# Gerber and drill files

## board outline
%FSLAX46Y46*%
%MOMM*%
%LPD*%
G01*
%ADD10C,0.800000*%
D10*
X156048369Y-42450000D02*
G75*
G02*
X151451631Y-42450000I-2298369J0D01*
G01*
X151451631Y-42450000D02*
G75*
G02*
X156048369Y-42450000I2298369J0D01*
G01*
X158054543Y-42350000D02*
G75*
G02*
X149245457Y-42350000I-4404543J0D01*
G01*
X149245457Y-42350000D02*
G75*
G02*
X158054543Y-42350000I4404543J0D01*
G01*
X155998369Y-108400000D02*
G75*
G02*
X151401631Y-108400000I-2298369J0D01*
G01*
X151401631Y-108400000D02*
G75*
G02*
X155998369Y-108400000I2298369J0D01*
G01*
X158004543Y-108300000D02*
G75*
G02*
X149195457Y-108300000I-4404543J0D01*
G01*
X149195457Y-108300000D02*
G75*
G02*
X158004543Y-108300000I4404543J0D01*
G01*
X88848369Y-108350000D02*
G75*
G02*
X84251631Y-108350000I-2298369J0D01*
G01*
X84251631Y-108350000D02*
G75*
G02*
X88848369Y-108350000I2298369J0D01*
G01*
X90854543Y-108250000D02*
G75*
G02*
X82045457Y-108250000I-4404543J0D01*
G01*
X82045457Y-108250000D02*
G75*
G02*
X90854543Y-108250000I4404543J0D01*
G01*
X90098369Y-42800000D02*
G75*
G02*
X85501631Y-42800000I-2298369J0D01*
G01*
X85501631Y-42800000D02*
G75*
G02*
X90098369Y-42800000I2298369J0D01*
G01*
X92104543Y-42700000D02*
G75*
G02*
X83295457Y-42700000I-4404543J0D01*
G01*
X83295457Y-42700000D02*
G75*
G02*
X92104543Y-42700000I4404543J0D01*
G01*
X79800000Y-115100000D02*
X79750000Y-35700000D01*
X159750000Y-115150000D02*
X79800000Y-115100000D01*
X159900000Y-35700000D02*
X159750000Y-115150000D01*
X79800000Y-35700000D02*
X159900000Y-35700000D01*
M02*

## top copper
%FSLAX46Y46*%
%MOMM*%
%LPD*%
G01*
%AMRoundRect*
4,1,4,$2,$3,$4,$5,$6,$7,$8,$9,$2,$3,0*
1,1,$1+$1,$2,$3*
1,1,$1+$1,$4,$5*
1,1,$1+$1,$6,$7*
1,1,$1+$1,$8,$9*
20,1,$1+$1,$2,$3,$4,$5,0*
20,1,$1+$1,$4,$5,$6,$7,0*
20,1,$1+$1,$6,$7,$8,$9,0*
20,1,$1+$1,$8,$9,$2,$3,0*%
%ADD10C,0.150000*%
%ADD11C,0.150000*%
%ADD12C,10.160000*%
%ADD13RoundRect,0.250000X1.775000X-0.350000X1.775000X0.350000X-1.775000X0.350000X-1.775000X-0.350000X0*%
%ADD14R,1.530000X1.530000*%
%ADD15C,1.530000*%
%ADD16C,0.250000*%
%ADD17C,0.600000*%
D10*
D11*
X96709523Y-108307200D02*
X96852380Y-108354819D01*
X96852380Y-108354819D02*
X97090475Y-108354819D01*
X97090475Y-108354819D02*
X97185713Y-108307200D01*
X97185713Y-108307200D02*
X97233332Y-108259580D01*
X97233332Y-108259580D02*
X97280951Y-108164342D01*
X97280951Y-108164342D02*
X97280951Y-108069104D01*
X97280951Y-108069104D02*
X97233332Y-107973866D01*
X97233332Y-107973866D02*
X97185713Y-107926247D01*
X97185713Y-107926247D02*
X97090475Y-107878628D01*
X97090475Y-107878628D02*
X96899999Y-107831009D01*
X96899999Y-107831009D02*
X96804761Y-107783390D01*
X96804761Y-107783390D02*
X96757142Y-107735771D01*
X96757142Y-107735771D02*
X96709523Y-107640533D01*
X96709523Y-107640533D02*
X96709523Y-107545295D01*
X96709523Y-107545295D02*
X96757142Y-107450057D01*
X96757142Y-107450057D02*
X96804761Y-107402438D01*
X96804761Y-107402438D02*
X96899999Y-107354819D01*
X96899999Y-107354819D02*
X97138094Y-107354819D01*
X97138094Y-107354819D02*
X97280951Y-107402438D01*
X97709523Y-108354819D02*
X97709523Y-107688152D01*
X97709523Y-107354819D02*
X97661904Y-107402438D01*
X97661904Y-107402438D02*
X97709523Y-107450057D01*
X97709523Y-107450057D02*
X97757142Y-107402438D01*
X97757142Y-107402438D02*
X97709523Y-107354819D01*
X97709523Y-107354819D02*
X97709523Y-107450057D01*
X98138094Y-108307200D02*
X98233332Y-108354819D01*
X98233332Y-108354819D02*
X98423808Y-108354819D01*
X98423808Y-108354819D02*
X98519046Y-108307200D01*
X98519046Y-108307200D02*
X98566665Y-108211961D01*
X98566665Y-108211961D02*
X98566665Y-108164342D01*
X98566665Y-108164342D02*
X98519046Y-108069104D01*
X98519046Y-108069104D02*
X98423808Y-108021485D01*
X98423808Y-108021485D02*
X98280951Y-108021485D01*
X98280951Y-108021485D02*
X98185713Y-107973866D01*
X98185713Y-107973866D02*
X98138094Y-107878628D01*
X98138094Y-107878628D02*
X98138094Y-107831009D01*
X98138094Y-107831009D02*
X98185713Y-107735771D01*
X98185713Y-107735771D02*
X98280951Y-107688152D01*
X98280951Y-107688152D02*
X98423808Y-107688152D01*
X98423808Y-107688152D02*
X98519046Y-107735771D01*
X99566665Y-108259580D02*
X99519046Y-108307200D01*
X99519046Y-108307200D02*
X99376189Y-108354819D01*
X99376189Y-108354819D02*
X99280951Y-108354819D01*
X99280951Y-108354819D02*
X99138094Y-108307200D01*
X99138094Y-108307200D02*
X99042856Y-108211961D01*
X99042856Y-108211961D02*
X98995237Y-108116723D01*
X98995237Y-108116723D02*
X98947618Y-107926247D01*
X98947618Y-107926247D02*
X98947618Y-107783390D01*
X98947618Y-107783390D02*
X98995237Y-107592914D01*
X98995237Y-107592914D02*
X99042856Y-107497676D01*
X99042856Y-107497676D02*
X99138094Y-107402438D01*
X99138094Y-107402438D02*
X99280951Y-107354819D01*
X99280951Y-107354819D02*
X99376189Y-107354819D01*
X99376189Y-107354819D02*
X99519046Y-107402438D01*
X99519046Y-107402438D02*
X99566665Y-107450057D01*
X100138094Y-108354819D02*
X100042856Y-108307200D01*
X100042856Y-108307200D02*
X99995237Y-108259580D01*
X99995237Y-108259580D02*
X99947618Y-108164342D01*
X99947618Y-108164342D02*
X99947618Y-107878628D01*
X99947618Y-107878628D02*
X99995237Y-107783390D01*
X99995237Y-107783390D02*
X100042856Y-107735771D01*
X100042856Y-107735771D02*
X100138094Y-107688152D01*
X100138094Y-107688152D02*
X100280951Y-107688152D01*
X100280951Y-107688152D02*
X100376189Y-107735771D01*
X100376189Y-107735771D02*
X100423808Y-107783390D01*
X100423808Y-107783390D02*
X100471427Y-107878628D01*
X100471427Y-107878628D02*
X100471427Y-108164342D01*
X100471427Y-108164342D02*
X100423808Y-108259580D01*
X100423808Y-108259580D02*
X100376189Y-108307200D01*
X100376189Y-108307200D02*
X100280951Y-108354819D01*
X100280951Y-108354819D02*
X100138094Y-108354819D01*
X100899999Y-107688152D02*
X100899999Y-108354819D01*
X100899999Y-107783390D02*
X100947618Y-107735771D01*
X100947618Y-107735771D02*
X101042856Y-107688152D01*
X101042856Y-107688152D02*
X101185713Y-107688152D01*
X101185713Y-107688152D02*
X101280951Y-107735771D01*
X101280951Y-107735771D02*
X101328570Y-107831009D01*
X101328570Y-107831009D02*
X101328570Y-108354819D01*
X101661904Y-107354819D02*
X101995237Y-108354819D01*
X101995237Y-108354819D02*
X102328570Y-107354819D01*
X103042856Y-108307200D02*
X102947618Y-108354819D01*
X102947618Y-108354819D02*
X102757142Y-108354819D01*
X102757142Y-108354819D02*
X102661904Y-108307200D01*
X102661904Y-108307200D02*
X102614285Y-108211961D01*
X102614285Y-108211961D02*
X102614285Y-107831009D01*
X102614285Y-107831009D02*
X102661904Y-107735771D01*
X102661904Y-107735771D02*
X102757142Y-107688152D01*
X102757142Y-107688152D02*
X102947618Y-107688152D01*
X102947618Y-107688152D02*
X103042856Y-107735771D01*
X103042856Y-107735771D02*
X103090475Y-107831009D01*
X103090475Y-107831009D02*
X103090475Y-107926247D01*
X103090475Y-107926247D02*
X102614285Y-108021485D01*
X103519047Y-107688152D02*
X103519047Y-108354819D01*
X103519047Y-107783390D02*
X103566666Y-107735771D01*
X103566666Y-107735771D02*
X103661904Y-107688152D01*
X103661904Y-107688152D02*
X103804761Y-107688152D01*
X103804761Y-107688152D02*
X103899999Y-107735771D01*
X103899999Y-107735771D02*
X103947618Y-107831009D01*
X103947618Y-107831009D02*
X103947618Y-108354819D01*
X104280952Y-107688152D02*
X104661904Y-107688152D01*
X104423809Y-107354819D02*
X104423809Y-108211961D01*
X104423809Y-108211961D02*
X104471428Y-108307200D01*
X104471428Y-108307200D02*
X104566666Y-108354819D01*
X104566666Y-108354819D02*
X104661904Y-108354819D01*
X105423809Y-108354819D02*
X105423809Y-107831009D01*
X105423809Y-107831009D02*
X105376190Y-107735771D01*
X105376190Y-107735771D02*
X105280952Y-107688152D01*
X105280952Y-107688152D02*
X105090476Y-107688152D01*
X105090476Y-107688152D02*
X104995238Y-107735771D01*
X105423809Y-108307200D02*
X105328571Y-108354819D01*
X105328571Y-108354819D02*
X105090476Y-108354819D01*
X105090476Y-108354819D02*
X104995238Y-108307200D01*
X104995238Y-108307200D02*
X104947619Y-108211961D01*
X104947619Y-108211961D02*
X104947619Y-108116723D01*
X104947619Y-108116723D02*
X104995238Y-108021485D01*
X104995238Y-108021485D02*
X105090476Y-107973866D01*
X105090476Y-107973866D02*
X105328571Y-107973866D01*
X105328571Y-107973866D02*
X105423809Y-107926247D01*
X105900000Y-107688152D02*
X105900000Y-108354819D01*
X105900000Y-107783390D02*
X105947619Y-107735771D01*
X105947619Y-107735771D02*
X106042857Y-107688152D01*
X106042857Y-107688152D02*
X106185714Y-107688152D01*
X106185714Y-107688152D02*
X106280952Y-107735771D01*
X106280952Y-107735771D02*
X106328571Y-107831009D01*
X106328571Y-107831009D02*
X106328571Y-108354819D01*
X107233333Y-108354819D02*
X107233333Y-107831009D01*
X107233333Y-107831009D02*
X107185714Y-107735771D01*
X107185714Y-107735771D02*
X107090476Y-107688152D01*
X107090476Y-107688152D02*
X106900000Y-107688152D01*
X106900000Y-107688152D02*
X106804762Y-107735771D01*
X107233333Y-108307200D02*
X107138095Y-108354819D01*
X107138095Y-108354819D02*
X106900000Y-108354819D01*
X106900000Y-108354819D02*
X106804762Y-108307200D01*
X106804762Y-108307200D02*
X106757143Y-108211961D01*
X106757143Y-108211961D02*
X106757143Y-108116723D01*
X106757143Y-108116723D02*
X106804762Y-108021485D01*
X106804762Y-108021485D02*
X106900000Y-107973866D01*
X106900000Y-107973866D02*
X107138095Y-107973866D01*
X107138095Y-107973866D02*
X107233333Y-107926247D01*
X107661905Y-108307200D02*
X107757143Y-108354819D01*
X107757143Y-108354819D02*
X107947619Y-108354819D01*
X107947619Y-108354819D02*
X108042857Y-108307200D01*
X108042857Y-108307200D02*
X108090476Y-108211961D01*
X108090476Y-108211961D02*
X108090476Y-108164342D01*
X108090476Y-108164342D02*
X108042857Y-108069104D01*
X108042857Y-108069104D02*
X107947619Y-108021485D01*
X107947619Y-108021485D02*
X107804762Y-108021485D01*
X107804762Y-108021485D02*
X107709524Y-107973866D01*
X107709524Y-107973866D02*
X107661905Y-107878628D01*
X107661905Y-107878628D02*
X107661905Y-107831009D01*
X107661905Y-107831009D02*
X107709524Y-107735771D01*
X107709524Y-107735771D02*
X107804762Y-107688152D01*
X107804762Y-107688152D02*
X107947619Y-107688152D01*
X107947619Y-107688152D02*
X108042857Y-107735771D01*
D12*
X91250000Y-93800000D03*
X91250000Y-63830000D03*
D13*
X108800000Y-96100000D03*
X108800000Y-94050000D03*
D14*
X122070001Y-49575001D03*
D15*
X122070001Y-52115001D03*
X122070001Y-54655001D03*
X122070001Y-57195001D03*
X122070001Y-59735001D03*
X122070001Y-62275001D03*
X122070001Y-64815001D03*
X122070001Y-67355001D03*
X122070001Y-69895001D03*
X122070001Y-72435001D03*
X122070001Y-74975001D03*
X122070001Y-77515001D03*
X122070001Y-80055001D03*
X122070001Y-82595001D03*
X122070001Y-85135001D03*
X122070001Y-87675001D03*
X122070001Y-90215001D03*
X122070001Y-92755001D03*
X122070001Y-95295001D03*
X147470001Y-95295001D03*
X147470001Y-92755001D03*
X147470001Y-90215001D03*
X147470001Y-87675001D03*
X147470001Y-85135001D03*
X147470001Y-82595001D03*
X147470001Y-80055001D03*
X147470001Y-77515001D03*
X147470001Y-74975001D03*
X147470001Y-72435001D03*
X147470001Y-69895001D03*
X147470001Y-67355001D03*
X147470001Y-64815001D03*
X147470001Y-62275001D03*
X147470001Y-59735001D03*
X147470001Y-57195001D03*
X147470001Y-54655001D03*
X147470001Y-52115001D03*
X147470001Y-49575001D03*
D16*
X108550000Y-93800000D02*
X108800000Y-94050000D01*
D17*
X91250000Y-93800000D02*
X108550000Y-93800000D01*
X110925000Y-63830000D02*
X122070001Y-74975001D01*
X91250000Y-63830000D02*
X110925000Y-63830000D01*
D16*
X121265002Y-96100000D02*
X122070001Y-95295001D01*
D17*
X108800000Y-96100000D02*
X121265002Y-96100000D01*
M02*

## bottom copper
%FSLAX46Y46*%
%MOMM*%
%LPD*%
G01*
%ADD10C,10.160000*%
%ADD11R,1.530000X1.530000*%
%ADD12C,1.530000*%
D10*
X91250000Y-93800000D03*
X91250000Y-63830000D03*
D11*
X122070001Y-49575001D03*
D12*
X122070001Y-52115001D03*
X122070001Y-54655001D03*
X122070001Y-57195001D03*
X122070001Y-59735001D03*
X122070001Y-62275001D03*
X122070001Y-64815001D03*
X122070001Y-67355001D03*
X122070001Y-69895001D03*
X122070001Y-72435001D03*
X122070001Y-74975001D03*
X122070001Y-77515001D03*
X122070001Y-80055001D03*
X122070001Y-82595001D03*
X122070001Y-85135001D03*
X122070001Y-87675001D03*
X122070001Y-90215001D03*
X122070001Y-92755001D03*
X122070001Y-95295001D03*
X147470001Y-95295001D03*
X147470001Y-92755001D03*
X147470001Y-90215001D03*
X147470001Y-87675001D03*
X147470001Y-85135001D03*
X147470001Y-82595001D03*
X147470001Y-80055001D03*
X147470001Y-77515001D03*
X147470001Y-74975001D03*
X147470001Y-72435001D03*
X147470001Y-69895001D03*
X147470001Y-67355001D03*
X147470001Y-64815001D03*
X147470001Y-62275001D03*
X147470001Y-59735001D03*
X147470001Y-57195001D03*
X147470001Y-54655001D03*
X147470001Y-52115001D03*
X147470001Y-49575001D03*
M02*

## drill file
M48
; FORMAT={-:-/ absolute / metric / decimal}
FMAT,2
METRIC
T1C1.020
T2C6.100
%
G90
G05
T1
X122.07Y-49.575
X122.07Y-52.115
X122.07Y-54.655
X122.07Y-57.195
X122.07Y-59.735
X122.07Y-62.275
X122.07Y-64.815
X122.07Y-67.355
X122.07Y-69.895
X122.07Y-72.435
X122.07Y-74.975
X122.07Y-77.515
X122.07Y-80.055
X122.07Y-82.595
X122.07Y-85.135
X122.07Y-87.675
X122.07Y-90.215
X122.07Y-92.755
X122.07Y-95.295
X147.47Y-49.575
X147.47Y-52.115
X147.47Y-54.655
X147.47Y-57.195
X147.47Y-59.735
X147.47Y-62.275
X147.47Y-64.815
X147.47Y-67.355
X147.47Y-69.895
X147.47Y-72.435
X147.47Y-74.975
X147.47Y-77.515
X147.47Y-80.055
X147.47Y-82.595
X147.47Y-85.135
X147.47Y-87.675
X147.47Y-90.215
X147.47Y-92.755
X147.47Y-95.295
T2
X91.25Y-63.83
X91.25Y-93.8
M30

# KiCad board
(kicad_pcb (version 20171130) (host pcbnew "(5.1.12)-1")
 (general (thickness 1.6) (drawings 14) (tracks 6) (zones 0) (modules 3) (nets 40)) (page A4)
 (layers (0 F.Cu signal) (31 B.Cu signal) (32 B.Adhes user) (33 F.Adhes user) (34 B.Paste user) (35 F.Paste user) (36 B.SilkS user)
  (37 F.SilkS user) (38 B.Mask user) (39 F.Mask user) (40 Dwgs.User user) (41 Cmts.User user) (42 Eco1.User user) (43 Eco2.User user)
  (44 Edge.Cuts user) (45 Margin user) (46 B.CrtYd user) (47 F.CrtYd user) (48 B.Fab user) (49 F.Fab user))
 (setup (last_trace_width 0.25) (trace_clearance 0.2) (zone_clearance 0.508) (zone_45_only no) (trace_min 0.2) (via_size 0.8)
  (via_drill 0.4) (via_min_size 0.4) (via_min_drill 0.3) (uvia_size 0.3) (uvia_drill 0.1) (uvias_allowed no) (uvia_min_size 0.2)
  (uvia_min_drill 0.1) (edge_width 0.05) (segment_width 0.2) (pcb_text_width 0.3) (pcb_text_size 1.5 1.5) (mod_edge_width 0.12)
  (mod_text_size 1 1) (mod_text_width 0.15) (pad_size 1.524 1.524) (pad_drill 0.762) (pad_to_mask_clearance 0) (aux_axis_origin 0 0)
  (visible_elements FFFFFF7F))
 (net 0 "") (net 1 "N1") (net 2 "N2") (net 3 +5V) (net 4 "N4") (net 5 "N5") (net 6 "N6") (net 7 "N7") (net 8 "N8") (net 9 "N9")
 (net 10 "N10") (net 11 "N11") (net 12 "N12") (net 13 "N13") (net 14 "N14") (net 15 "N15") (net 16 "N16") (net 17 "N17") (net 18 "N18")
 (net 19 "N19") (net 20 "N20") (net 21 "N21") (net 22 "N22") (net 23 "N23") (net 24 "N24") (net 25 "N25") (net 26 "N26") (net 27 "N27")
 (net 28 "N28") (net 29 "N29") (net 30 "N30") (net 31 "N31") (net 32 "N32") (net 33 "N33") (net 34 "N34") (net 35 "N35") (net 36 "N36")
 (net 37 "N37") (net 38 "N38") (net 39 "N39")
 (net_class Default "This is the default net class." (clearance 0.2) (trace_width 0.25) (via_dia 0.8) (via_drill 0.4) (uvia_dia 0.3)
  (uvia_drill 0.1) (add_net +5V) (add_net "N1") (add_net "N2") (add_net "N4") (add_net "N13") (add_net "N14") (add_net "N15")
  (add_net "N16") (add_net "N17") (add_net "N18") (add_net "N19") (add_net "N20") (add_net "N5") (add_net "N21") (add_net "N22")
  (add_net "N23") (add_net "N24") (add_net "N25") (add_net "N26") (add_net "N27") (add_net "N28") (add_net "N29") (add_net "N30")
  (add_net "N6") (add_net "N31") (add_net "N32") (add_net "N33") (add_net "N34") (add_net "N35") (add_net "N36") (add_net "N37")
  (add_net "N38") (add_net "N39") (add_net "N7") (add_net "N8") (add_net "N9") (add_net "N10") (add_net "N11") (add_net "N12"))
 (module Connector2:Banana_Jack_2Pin (layer F.Cu) (at 91.25 93.8 90)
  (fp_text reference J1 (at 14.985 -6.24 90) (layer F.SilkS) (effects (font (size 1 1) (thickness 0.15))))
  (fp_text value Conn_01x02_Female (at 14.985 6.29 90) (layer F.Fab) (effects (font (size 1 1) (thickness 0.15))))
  (pad 1 thru_hole circle (at 0 0 90) (size 10.16 10.16) (drill 6.1) (layers *.Cu *.Mask) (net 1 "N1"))
  (pad 2 thru_hole circle (at 29.97 0 90) (size 10.16 10.16) (drill 6.1) (layers *.Cu *.Mask) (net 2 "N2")))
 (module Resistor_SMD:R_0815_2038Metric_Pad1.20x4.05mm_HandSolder (layer F.Cu) (at 108.8 95.075 90)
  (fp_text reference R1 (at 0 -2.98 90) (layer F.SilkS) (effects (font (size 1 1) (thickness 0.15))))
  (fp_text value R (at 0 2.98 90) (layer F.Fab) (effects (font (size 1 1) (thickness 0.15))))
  (pad 1 smd roundrect (at -1.025 0 90) (size 1.2 4.05) (layers F.Cu F.Paste F.Mask) (roundrect_rratio 0.208333) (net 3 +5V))
  (pad 2 smd roundrect (at 1.025 0 90) (size 1.2 4.05) (layers F.Cu F.Paste F.Mask) (roundrect_rratio 0.208333) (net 1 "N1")))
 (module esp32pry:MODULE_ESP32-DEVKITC (layer F.Cu) (at 134.770001 72.425001)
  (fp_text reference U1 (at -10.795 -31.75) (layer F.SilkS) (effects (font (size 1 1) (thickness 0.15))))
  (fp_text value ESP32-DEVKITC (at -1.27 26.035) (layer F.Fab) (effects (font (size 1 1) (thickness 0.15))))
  (pad 1 thru_hole rect (at -12.7 -22.85) (size 1.53 1.53) (drill 1.02) (layers *.Cu *.Mask) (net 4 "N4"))
  (pad 2 thru_hole circle (at -12.7 -20.31) (size 1.53 1.53) (drill 1.02) (layers *.Cu *.Mask) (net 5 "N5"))
  (pad 3 thru_hole circle (at -12.7 -17.77) (size 1.53 1.53) (drill 1.02) (layers *.Cu *.Mask) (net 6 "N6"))
  (pad 4 thru_hole circle (at -12.7 -15.23) (size 1.53 1.53) (drill 1.02) (layers *.Cu *.Mask) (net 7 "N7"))
  (pad 5 thru_hole circle (at -12.7 -12.69) (size 1.53 1.53) (drill 1.02) (layers *.Cu *.Mask) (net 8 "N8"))
  (pad 6 thru_hole circle (at -12.7 -10.15) (size 1.53 1.53) (drill 1.02) (layers *.Cu *.Mask) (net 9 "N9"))
  (pad 7 thru_hole circle (at -12.7 -7.61) (size 1.53 1.53) (drill 1.02) (layers *.Cu *.Mask) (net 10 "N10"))
  (pad 8 thru_hole circle (at -12.7 -5.07) (size 1.53 1.53) (drill 1.02) (layers *.Cu *.Mask) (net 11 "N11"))
  (pad 9 thru_hole circle (at -12.7 -2.53) (size 1.53 1.53) (drill 1.02) (layers *.Cu *.Mask) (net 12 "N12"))
  (pad 10 thru_hole circle (at -12.7 0.01) (size 1.53 1.53) (drill 1.02) (layers *.Cu *.Mask) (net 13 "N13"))
  (pad 11 thru_hole circle (at -12.7 2.55) (size 1.53 1.53) (drill 1.02) (layers *.Cu *.Mask) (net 2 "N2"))
  (pad 12 thru_hole circle (at -12.7 5.09) (size 1.53 1.53) (drill 1.02) (layers *.Cu *.Mask) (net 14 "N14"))
  (pad 13 thru_hole circle (at -12.7 7.63) (size 1.53 1.53) (drill 1.02) (layers *.Cu *.Mask) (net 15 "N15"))
  (pad 14 thru_hole circle (at -12.7 10.17) (size 1.53 1.53) (drill 1.02) (layers *.Cu *.Mask) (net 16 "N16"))
  (pad 15 thru_hole circle (at -12.7 12.71) (size 1.53 1.53) (drill 1.02) (layers *.Cu *.Mask) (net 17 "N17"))
  (pad 16 thru_hole circle (at -12.7 15.25) (size 1.53 1.53) (drill 1.02) (layers *.Cu *.Mask) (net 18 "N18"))
  (pad 17 thru_hole circle (at -12.7 17.79) (size 1.53 1.53) (drill 1.02) (layers *.Cu *.Mask) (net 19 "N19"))
  (pad 18 thru_hole circle (at -12.7 20.33) (size 1.53 1.53) (drill 1.02) (layers *.Cu *.Mask) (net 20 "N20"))
  (pad 19 thru_hole circle (at -12.7 22.87) (size 1.53 1.53) (drill 1.02) (layers *.Cu *.Mask) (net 3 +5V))
  (pad 20 thru_hole circle (at 12.7 22.87) (size 1.53 1.53) (drill 1.02) (layers *.Cu *.Mask) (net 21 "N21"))
  (pad 21 thru_hole circle (at 12.7 20.33) (size 1.53 1.53) (drill 1.02) (layers *.Cu *.Mask) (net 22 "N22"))
  (pad 22 thru_hole circle (at 12.7 17.79) (size 1.53 1.53) (drill 1.02) (layers *.Cu *.Mask) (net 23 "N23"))
  (pad 23 thru_hole circle (at 12.7 15.25) (size 1.53 1.53) (drill 1.02) (layers *.Cu *.Mask) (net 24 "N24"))
  (pad 24 thru_hole circle (at 12.7 12.71) (size 1.53 1.53) (drill 1.02) (layers *.Cu *.Mask) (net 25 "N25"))
  (pad 25 thru_hole circle (at 12.7 10.17) (size 1.53 1.53) (drill 1.02) (layers *.Cu *.Mask) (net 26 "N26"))
  (pad 26 thru_hole circle (at 12.7 7.63) (size 1.53 1.53) (drill 1.02) (layers *.Cu *.Mask) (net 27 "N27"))
  (pad 27 thru_hole circle (at 12.7 5.09) (size 1.53 1.53) (drill 1.02) (layers *.Cu *.Mask) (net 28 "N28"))
  (pad 28 thru_hole circle (at 12.7 2.55) (size 1.53 1.53) (drill 1.02) (layers *.Cu *.Mask) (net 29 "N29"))
  (pad 29 thru_hole circle (at 12.7 0.01) (size 1.53 1.53) (drill 1.02) (layers *.Cu *.Mask) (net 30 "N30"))
  (pad 30 thru_hole circle (at 12.7 -2.53) (size 1.53 1.53) (drill 1.02) (layers *.Cu *.Mask) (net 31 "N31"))
  (pad 31 thru_hole circle (at 12.7 -5.07) (size 1.53 1.53) (drill 1.02) (layers *.Cu *.Mask) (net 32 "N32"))
  (pad 32 thru_hole circle (at 12.7 -7.61) (size 1.53 1.53) (drill 1.02) (layers *.Cu *.Mask) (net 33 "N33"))
  (pad 33 thru_hole circle (at 12.7 -10.15) (size 1.53 1.53) (drill 1.02) (layers *.Cu *.Mask) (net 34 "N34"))
  (pad 34 thru_hole circle (at 12.7 -12.69) (size 1.53 1.53) (drill 1.02) (layers *.Cu *.Mask) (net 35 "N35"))
  (pad 35 thru_hole circle (at 12.7 -15.23) (size 1.53 1.53) (drill 1.02) (layers *.Cu *.Mask) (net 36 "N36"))
  (pad 36 thru_hole circle (at 12.7 -17.77) (size 1.53 1.53) (drill 1.02) (layers *.Cu *.Mask) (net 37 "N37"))
  (pad 37 thru_hole circle (at 12.7 -20.31) (size 1.53 1.53) (drill 1.02) (layers *.Cu *.Mask) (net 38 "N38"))
  (pad 38 thru_hole circle (at 12.7 -22.85) (size 1.53 1.53) (drill 1.02) (layers *.Cu *.Mask) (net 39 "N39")))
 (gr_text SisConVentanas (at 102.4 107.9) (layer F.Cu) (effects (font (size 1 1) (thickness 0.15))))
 (gr_circle (center 153.75 42.45) (end 156.048369 42.45) (layer Edge.Cuts) (width 0.8))
 (gr_circle (center 153.65 42.35) (end 158.054543 42.35) (layer Edge.Cuts) (width 0.8))
 (gr_circle (center 153.7 108.4) (end 155.998369 108.4) (layer Edge.Cuts) (width 0.8))
 (gr_circle (center 153.6 108.3) (end 158.004543 108.3) (layer Edge.Cuts) (width 0.8))
 (gr_circle (center 86.55 108.35) (end 88.848369 108.35) (layer Edge.Cuts) (width 0.8))
 (gr_circle (center 86.45 108.25) (end 90.854543 108.25) (layer Edge.Cuts) (width 0.8))
 (gr_circle (center 87.8 42.8) (end 90.098369 42.8) (layer Edge.Cuts) (width 0.8))
 (gr_circle (center 87.7 42.7) (end 92.104543 42.7) (layer Edge.Cuts) (width 0.8))
 (gr_line (start 79.8 115.1) (end 79.75 35.7) (layer Edge.Cuts) (width 0.8))
 (gr_line (start 159.75 115.15) (end 79.8 115.1) (layer Edge.Cuts) (width 0.8))
 (gr_line (start 159.9 35.7) (end 159.75 115.15) (layer Edge.Cuts) (width 0.8))
 (gr_line (start 79.8 35.7) (end 159.9 35.7) (layer Edge.Cuts) (width 0.8))
 (segment (start 108.55 93.8) (end 108.8 94.05) (width 0.25) (layer F.Cu) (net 1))
 (segment (start 91.25 93.8) (end 108.55 93.8) (width 0.6) (layer F.Cu) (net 1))
 (segment (start 110.925 63.83) (end 122.070001 74.975001) (width 0.6) (layer F.Cu) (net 2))
 (segment (start 91.25 63.83) (end 110.925 63.83) (width 0.6) (layer F.Cu) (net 2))
 (segment (start 121.265002 96.1) (end 122.070001 95.295001) (width 0.25) (layer F.Cu) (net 3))
 (segment (start 108.8 96.1) (end 121.265002 96.1) (width 0.6) (layer F.Cu) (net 3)))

